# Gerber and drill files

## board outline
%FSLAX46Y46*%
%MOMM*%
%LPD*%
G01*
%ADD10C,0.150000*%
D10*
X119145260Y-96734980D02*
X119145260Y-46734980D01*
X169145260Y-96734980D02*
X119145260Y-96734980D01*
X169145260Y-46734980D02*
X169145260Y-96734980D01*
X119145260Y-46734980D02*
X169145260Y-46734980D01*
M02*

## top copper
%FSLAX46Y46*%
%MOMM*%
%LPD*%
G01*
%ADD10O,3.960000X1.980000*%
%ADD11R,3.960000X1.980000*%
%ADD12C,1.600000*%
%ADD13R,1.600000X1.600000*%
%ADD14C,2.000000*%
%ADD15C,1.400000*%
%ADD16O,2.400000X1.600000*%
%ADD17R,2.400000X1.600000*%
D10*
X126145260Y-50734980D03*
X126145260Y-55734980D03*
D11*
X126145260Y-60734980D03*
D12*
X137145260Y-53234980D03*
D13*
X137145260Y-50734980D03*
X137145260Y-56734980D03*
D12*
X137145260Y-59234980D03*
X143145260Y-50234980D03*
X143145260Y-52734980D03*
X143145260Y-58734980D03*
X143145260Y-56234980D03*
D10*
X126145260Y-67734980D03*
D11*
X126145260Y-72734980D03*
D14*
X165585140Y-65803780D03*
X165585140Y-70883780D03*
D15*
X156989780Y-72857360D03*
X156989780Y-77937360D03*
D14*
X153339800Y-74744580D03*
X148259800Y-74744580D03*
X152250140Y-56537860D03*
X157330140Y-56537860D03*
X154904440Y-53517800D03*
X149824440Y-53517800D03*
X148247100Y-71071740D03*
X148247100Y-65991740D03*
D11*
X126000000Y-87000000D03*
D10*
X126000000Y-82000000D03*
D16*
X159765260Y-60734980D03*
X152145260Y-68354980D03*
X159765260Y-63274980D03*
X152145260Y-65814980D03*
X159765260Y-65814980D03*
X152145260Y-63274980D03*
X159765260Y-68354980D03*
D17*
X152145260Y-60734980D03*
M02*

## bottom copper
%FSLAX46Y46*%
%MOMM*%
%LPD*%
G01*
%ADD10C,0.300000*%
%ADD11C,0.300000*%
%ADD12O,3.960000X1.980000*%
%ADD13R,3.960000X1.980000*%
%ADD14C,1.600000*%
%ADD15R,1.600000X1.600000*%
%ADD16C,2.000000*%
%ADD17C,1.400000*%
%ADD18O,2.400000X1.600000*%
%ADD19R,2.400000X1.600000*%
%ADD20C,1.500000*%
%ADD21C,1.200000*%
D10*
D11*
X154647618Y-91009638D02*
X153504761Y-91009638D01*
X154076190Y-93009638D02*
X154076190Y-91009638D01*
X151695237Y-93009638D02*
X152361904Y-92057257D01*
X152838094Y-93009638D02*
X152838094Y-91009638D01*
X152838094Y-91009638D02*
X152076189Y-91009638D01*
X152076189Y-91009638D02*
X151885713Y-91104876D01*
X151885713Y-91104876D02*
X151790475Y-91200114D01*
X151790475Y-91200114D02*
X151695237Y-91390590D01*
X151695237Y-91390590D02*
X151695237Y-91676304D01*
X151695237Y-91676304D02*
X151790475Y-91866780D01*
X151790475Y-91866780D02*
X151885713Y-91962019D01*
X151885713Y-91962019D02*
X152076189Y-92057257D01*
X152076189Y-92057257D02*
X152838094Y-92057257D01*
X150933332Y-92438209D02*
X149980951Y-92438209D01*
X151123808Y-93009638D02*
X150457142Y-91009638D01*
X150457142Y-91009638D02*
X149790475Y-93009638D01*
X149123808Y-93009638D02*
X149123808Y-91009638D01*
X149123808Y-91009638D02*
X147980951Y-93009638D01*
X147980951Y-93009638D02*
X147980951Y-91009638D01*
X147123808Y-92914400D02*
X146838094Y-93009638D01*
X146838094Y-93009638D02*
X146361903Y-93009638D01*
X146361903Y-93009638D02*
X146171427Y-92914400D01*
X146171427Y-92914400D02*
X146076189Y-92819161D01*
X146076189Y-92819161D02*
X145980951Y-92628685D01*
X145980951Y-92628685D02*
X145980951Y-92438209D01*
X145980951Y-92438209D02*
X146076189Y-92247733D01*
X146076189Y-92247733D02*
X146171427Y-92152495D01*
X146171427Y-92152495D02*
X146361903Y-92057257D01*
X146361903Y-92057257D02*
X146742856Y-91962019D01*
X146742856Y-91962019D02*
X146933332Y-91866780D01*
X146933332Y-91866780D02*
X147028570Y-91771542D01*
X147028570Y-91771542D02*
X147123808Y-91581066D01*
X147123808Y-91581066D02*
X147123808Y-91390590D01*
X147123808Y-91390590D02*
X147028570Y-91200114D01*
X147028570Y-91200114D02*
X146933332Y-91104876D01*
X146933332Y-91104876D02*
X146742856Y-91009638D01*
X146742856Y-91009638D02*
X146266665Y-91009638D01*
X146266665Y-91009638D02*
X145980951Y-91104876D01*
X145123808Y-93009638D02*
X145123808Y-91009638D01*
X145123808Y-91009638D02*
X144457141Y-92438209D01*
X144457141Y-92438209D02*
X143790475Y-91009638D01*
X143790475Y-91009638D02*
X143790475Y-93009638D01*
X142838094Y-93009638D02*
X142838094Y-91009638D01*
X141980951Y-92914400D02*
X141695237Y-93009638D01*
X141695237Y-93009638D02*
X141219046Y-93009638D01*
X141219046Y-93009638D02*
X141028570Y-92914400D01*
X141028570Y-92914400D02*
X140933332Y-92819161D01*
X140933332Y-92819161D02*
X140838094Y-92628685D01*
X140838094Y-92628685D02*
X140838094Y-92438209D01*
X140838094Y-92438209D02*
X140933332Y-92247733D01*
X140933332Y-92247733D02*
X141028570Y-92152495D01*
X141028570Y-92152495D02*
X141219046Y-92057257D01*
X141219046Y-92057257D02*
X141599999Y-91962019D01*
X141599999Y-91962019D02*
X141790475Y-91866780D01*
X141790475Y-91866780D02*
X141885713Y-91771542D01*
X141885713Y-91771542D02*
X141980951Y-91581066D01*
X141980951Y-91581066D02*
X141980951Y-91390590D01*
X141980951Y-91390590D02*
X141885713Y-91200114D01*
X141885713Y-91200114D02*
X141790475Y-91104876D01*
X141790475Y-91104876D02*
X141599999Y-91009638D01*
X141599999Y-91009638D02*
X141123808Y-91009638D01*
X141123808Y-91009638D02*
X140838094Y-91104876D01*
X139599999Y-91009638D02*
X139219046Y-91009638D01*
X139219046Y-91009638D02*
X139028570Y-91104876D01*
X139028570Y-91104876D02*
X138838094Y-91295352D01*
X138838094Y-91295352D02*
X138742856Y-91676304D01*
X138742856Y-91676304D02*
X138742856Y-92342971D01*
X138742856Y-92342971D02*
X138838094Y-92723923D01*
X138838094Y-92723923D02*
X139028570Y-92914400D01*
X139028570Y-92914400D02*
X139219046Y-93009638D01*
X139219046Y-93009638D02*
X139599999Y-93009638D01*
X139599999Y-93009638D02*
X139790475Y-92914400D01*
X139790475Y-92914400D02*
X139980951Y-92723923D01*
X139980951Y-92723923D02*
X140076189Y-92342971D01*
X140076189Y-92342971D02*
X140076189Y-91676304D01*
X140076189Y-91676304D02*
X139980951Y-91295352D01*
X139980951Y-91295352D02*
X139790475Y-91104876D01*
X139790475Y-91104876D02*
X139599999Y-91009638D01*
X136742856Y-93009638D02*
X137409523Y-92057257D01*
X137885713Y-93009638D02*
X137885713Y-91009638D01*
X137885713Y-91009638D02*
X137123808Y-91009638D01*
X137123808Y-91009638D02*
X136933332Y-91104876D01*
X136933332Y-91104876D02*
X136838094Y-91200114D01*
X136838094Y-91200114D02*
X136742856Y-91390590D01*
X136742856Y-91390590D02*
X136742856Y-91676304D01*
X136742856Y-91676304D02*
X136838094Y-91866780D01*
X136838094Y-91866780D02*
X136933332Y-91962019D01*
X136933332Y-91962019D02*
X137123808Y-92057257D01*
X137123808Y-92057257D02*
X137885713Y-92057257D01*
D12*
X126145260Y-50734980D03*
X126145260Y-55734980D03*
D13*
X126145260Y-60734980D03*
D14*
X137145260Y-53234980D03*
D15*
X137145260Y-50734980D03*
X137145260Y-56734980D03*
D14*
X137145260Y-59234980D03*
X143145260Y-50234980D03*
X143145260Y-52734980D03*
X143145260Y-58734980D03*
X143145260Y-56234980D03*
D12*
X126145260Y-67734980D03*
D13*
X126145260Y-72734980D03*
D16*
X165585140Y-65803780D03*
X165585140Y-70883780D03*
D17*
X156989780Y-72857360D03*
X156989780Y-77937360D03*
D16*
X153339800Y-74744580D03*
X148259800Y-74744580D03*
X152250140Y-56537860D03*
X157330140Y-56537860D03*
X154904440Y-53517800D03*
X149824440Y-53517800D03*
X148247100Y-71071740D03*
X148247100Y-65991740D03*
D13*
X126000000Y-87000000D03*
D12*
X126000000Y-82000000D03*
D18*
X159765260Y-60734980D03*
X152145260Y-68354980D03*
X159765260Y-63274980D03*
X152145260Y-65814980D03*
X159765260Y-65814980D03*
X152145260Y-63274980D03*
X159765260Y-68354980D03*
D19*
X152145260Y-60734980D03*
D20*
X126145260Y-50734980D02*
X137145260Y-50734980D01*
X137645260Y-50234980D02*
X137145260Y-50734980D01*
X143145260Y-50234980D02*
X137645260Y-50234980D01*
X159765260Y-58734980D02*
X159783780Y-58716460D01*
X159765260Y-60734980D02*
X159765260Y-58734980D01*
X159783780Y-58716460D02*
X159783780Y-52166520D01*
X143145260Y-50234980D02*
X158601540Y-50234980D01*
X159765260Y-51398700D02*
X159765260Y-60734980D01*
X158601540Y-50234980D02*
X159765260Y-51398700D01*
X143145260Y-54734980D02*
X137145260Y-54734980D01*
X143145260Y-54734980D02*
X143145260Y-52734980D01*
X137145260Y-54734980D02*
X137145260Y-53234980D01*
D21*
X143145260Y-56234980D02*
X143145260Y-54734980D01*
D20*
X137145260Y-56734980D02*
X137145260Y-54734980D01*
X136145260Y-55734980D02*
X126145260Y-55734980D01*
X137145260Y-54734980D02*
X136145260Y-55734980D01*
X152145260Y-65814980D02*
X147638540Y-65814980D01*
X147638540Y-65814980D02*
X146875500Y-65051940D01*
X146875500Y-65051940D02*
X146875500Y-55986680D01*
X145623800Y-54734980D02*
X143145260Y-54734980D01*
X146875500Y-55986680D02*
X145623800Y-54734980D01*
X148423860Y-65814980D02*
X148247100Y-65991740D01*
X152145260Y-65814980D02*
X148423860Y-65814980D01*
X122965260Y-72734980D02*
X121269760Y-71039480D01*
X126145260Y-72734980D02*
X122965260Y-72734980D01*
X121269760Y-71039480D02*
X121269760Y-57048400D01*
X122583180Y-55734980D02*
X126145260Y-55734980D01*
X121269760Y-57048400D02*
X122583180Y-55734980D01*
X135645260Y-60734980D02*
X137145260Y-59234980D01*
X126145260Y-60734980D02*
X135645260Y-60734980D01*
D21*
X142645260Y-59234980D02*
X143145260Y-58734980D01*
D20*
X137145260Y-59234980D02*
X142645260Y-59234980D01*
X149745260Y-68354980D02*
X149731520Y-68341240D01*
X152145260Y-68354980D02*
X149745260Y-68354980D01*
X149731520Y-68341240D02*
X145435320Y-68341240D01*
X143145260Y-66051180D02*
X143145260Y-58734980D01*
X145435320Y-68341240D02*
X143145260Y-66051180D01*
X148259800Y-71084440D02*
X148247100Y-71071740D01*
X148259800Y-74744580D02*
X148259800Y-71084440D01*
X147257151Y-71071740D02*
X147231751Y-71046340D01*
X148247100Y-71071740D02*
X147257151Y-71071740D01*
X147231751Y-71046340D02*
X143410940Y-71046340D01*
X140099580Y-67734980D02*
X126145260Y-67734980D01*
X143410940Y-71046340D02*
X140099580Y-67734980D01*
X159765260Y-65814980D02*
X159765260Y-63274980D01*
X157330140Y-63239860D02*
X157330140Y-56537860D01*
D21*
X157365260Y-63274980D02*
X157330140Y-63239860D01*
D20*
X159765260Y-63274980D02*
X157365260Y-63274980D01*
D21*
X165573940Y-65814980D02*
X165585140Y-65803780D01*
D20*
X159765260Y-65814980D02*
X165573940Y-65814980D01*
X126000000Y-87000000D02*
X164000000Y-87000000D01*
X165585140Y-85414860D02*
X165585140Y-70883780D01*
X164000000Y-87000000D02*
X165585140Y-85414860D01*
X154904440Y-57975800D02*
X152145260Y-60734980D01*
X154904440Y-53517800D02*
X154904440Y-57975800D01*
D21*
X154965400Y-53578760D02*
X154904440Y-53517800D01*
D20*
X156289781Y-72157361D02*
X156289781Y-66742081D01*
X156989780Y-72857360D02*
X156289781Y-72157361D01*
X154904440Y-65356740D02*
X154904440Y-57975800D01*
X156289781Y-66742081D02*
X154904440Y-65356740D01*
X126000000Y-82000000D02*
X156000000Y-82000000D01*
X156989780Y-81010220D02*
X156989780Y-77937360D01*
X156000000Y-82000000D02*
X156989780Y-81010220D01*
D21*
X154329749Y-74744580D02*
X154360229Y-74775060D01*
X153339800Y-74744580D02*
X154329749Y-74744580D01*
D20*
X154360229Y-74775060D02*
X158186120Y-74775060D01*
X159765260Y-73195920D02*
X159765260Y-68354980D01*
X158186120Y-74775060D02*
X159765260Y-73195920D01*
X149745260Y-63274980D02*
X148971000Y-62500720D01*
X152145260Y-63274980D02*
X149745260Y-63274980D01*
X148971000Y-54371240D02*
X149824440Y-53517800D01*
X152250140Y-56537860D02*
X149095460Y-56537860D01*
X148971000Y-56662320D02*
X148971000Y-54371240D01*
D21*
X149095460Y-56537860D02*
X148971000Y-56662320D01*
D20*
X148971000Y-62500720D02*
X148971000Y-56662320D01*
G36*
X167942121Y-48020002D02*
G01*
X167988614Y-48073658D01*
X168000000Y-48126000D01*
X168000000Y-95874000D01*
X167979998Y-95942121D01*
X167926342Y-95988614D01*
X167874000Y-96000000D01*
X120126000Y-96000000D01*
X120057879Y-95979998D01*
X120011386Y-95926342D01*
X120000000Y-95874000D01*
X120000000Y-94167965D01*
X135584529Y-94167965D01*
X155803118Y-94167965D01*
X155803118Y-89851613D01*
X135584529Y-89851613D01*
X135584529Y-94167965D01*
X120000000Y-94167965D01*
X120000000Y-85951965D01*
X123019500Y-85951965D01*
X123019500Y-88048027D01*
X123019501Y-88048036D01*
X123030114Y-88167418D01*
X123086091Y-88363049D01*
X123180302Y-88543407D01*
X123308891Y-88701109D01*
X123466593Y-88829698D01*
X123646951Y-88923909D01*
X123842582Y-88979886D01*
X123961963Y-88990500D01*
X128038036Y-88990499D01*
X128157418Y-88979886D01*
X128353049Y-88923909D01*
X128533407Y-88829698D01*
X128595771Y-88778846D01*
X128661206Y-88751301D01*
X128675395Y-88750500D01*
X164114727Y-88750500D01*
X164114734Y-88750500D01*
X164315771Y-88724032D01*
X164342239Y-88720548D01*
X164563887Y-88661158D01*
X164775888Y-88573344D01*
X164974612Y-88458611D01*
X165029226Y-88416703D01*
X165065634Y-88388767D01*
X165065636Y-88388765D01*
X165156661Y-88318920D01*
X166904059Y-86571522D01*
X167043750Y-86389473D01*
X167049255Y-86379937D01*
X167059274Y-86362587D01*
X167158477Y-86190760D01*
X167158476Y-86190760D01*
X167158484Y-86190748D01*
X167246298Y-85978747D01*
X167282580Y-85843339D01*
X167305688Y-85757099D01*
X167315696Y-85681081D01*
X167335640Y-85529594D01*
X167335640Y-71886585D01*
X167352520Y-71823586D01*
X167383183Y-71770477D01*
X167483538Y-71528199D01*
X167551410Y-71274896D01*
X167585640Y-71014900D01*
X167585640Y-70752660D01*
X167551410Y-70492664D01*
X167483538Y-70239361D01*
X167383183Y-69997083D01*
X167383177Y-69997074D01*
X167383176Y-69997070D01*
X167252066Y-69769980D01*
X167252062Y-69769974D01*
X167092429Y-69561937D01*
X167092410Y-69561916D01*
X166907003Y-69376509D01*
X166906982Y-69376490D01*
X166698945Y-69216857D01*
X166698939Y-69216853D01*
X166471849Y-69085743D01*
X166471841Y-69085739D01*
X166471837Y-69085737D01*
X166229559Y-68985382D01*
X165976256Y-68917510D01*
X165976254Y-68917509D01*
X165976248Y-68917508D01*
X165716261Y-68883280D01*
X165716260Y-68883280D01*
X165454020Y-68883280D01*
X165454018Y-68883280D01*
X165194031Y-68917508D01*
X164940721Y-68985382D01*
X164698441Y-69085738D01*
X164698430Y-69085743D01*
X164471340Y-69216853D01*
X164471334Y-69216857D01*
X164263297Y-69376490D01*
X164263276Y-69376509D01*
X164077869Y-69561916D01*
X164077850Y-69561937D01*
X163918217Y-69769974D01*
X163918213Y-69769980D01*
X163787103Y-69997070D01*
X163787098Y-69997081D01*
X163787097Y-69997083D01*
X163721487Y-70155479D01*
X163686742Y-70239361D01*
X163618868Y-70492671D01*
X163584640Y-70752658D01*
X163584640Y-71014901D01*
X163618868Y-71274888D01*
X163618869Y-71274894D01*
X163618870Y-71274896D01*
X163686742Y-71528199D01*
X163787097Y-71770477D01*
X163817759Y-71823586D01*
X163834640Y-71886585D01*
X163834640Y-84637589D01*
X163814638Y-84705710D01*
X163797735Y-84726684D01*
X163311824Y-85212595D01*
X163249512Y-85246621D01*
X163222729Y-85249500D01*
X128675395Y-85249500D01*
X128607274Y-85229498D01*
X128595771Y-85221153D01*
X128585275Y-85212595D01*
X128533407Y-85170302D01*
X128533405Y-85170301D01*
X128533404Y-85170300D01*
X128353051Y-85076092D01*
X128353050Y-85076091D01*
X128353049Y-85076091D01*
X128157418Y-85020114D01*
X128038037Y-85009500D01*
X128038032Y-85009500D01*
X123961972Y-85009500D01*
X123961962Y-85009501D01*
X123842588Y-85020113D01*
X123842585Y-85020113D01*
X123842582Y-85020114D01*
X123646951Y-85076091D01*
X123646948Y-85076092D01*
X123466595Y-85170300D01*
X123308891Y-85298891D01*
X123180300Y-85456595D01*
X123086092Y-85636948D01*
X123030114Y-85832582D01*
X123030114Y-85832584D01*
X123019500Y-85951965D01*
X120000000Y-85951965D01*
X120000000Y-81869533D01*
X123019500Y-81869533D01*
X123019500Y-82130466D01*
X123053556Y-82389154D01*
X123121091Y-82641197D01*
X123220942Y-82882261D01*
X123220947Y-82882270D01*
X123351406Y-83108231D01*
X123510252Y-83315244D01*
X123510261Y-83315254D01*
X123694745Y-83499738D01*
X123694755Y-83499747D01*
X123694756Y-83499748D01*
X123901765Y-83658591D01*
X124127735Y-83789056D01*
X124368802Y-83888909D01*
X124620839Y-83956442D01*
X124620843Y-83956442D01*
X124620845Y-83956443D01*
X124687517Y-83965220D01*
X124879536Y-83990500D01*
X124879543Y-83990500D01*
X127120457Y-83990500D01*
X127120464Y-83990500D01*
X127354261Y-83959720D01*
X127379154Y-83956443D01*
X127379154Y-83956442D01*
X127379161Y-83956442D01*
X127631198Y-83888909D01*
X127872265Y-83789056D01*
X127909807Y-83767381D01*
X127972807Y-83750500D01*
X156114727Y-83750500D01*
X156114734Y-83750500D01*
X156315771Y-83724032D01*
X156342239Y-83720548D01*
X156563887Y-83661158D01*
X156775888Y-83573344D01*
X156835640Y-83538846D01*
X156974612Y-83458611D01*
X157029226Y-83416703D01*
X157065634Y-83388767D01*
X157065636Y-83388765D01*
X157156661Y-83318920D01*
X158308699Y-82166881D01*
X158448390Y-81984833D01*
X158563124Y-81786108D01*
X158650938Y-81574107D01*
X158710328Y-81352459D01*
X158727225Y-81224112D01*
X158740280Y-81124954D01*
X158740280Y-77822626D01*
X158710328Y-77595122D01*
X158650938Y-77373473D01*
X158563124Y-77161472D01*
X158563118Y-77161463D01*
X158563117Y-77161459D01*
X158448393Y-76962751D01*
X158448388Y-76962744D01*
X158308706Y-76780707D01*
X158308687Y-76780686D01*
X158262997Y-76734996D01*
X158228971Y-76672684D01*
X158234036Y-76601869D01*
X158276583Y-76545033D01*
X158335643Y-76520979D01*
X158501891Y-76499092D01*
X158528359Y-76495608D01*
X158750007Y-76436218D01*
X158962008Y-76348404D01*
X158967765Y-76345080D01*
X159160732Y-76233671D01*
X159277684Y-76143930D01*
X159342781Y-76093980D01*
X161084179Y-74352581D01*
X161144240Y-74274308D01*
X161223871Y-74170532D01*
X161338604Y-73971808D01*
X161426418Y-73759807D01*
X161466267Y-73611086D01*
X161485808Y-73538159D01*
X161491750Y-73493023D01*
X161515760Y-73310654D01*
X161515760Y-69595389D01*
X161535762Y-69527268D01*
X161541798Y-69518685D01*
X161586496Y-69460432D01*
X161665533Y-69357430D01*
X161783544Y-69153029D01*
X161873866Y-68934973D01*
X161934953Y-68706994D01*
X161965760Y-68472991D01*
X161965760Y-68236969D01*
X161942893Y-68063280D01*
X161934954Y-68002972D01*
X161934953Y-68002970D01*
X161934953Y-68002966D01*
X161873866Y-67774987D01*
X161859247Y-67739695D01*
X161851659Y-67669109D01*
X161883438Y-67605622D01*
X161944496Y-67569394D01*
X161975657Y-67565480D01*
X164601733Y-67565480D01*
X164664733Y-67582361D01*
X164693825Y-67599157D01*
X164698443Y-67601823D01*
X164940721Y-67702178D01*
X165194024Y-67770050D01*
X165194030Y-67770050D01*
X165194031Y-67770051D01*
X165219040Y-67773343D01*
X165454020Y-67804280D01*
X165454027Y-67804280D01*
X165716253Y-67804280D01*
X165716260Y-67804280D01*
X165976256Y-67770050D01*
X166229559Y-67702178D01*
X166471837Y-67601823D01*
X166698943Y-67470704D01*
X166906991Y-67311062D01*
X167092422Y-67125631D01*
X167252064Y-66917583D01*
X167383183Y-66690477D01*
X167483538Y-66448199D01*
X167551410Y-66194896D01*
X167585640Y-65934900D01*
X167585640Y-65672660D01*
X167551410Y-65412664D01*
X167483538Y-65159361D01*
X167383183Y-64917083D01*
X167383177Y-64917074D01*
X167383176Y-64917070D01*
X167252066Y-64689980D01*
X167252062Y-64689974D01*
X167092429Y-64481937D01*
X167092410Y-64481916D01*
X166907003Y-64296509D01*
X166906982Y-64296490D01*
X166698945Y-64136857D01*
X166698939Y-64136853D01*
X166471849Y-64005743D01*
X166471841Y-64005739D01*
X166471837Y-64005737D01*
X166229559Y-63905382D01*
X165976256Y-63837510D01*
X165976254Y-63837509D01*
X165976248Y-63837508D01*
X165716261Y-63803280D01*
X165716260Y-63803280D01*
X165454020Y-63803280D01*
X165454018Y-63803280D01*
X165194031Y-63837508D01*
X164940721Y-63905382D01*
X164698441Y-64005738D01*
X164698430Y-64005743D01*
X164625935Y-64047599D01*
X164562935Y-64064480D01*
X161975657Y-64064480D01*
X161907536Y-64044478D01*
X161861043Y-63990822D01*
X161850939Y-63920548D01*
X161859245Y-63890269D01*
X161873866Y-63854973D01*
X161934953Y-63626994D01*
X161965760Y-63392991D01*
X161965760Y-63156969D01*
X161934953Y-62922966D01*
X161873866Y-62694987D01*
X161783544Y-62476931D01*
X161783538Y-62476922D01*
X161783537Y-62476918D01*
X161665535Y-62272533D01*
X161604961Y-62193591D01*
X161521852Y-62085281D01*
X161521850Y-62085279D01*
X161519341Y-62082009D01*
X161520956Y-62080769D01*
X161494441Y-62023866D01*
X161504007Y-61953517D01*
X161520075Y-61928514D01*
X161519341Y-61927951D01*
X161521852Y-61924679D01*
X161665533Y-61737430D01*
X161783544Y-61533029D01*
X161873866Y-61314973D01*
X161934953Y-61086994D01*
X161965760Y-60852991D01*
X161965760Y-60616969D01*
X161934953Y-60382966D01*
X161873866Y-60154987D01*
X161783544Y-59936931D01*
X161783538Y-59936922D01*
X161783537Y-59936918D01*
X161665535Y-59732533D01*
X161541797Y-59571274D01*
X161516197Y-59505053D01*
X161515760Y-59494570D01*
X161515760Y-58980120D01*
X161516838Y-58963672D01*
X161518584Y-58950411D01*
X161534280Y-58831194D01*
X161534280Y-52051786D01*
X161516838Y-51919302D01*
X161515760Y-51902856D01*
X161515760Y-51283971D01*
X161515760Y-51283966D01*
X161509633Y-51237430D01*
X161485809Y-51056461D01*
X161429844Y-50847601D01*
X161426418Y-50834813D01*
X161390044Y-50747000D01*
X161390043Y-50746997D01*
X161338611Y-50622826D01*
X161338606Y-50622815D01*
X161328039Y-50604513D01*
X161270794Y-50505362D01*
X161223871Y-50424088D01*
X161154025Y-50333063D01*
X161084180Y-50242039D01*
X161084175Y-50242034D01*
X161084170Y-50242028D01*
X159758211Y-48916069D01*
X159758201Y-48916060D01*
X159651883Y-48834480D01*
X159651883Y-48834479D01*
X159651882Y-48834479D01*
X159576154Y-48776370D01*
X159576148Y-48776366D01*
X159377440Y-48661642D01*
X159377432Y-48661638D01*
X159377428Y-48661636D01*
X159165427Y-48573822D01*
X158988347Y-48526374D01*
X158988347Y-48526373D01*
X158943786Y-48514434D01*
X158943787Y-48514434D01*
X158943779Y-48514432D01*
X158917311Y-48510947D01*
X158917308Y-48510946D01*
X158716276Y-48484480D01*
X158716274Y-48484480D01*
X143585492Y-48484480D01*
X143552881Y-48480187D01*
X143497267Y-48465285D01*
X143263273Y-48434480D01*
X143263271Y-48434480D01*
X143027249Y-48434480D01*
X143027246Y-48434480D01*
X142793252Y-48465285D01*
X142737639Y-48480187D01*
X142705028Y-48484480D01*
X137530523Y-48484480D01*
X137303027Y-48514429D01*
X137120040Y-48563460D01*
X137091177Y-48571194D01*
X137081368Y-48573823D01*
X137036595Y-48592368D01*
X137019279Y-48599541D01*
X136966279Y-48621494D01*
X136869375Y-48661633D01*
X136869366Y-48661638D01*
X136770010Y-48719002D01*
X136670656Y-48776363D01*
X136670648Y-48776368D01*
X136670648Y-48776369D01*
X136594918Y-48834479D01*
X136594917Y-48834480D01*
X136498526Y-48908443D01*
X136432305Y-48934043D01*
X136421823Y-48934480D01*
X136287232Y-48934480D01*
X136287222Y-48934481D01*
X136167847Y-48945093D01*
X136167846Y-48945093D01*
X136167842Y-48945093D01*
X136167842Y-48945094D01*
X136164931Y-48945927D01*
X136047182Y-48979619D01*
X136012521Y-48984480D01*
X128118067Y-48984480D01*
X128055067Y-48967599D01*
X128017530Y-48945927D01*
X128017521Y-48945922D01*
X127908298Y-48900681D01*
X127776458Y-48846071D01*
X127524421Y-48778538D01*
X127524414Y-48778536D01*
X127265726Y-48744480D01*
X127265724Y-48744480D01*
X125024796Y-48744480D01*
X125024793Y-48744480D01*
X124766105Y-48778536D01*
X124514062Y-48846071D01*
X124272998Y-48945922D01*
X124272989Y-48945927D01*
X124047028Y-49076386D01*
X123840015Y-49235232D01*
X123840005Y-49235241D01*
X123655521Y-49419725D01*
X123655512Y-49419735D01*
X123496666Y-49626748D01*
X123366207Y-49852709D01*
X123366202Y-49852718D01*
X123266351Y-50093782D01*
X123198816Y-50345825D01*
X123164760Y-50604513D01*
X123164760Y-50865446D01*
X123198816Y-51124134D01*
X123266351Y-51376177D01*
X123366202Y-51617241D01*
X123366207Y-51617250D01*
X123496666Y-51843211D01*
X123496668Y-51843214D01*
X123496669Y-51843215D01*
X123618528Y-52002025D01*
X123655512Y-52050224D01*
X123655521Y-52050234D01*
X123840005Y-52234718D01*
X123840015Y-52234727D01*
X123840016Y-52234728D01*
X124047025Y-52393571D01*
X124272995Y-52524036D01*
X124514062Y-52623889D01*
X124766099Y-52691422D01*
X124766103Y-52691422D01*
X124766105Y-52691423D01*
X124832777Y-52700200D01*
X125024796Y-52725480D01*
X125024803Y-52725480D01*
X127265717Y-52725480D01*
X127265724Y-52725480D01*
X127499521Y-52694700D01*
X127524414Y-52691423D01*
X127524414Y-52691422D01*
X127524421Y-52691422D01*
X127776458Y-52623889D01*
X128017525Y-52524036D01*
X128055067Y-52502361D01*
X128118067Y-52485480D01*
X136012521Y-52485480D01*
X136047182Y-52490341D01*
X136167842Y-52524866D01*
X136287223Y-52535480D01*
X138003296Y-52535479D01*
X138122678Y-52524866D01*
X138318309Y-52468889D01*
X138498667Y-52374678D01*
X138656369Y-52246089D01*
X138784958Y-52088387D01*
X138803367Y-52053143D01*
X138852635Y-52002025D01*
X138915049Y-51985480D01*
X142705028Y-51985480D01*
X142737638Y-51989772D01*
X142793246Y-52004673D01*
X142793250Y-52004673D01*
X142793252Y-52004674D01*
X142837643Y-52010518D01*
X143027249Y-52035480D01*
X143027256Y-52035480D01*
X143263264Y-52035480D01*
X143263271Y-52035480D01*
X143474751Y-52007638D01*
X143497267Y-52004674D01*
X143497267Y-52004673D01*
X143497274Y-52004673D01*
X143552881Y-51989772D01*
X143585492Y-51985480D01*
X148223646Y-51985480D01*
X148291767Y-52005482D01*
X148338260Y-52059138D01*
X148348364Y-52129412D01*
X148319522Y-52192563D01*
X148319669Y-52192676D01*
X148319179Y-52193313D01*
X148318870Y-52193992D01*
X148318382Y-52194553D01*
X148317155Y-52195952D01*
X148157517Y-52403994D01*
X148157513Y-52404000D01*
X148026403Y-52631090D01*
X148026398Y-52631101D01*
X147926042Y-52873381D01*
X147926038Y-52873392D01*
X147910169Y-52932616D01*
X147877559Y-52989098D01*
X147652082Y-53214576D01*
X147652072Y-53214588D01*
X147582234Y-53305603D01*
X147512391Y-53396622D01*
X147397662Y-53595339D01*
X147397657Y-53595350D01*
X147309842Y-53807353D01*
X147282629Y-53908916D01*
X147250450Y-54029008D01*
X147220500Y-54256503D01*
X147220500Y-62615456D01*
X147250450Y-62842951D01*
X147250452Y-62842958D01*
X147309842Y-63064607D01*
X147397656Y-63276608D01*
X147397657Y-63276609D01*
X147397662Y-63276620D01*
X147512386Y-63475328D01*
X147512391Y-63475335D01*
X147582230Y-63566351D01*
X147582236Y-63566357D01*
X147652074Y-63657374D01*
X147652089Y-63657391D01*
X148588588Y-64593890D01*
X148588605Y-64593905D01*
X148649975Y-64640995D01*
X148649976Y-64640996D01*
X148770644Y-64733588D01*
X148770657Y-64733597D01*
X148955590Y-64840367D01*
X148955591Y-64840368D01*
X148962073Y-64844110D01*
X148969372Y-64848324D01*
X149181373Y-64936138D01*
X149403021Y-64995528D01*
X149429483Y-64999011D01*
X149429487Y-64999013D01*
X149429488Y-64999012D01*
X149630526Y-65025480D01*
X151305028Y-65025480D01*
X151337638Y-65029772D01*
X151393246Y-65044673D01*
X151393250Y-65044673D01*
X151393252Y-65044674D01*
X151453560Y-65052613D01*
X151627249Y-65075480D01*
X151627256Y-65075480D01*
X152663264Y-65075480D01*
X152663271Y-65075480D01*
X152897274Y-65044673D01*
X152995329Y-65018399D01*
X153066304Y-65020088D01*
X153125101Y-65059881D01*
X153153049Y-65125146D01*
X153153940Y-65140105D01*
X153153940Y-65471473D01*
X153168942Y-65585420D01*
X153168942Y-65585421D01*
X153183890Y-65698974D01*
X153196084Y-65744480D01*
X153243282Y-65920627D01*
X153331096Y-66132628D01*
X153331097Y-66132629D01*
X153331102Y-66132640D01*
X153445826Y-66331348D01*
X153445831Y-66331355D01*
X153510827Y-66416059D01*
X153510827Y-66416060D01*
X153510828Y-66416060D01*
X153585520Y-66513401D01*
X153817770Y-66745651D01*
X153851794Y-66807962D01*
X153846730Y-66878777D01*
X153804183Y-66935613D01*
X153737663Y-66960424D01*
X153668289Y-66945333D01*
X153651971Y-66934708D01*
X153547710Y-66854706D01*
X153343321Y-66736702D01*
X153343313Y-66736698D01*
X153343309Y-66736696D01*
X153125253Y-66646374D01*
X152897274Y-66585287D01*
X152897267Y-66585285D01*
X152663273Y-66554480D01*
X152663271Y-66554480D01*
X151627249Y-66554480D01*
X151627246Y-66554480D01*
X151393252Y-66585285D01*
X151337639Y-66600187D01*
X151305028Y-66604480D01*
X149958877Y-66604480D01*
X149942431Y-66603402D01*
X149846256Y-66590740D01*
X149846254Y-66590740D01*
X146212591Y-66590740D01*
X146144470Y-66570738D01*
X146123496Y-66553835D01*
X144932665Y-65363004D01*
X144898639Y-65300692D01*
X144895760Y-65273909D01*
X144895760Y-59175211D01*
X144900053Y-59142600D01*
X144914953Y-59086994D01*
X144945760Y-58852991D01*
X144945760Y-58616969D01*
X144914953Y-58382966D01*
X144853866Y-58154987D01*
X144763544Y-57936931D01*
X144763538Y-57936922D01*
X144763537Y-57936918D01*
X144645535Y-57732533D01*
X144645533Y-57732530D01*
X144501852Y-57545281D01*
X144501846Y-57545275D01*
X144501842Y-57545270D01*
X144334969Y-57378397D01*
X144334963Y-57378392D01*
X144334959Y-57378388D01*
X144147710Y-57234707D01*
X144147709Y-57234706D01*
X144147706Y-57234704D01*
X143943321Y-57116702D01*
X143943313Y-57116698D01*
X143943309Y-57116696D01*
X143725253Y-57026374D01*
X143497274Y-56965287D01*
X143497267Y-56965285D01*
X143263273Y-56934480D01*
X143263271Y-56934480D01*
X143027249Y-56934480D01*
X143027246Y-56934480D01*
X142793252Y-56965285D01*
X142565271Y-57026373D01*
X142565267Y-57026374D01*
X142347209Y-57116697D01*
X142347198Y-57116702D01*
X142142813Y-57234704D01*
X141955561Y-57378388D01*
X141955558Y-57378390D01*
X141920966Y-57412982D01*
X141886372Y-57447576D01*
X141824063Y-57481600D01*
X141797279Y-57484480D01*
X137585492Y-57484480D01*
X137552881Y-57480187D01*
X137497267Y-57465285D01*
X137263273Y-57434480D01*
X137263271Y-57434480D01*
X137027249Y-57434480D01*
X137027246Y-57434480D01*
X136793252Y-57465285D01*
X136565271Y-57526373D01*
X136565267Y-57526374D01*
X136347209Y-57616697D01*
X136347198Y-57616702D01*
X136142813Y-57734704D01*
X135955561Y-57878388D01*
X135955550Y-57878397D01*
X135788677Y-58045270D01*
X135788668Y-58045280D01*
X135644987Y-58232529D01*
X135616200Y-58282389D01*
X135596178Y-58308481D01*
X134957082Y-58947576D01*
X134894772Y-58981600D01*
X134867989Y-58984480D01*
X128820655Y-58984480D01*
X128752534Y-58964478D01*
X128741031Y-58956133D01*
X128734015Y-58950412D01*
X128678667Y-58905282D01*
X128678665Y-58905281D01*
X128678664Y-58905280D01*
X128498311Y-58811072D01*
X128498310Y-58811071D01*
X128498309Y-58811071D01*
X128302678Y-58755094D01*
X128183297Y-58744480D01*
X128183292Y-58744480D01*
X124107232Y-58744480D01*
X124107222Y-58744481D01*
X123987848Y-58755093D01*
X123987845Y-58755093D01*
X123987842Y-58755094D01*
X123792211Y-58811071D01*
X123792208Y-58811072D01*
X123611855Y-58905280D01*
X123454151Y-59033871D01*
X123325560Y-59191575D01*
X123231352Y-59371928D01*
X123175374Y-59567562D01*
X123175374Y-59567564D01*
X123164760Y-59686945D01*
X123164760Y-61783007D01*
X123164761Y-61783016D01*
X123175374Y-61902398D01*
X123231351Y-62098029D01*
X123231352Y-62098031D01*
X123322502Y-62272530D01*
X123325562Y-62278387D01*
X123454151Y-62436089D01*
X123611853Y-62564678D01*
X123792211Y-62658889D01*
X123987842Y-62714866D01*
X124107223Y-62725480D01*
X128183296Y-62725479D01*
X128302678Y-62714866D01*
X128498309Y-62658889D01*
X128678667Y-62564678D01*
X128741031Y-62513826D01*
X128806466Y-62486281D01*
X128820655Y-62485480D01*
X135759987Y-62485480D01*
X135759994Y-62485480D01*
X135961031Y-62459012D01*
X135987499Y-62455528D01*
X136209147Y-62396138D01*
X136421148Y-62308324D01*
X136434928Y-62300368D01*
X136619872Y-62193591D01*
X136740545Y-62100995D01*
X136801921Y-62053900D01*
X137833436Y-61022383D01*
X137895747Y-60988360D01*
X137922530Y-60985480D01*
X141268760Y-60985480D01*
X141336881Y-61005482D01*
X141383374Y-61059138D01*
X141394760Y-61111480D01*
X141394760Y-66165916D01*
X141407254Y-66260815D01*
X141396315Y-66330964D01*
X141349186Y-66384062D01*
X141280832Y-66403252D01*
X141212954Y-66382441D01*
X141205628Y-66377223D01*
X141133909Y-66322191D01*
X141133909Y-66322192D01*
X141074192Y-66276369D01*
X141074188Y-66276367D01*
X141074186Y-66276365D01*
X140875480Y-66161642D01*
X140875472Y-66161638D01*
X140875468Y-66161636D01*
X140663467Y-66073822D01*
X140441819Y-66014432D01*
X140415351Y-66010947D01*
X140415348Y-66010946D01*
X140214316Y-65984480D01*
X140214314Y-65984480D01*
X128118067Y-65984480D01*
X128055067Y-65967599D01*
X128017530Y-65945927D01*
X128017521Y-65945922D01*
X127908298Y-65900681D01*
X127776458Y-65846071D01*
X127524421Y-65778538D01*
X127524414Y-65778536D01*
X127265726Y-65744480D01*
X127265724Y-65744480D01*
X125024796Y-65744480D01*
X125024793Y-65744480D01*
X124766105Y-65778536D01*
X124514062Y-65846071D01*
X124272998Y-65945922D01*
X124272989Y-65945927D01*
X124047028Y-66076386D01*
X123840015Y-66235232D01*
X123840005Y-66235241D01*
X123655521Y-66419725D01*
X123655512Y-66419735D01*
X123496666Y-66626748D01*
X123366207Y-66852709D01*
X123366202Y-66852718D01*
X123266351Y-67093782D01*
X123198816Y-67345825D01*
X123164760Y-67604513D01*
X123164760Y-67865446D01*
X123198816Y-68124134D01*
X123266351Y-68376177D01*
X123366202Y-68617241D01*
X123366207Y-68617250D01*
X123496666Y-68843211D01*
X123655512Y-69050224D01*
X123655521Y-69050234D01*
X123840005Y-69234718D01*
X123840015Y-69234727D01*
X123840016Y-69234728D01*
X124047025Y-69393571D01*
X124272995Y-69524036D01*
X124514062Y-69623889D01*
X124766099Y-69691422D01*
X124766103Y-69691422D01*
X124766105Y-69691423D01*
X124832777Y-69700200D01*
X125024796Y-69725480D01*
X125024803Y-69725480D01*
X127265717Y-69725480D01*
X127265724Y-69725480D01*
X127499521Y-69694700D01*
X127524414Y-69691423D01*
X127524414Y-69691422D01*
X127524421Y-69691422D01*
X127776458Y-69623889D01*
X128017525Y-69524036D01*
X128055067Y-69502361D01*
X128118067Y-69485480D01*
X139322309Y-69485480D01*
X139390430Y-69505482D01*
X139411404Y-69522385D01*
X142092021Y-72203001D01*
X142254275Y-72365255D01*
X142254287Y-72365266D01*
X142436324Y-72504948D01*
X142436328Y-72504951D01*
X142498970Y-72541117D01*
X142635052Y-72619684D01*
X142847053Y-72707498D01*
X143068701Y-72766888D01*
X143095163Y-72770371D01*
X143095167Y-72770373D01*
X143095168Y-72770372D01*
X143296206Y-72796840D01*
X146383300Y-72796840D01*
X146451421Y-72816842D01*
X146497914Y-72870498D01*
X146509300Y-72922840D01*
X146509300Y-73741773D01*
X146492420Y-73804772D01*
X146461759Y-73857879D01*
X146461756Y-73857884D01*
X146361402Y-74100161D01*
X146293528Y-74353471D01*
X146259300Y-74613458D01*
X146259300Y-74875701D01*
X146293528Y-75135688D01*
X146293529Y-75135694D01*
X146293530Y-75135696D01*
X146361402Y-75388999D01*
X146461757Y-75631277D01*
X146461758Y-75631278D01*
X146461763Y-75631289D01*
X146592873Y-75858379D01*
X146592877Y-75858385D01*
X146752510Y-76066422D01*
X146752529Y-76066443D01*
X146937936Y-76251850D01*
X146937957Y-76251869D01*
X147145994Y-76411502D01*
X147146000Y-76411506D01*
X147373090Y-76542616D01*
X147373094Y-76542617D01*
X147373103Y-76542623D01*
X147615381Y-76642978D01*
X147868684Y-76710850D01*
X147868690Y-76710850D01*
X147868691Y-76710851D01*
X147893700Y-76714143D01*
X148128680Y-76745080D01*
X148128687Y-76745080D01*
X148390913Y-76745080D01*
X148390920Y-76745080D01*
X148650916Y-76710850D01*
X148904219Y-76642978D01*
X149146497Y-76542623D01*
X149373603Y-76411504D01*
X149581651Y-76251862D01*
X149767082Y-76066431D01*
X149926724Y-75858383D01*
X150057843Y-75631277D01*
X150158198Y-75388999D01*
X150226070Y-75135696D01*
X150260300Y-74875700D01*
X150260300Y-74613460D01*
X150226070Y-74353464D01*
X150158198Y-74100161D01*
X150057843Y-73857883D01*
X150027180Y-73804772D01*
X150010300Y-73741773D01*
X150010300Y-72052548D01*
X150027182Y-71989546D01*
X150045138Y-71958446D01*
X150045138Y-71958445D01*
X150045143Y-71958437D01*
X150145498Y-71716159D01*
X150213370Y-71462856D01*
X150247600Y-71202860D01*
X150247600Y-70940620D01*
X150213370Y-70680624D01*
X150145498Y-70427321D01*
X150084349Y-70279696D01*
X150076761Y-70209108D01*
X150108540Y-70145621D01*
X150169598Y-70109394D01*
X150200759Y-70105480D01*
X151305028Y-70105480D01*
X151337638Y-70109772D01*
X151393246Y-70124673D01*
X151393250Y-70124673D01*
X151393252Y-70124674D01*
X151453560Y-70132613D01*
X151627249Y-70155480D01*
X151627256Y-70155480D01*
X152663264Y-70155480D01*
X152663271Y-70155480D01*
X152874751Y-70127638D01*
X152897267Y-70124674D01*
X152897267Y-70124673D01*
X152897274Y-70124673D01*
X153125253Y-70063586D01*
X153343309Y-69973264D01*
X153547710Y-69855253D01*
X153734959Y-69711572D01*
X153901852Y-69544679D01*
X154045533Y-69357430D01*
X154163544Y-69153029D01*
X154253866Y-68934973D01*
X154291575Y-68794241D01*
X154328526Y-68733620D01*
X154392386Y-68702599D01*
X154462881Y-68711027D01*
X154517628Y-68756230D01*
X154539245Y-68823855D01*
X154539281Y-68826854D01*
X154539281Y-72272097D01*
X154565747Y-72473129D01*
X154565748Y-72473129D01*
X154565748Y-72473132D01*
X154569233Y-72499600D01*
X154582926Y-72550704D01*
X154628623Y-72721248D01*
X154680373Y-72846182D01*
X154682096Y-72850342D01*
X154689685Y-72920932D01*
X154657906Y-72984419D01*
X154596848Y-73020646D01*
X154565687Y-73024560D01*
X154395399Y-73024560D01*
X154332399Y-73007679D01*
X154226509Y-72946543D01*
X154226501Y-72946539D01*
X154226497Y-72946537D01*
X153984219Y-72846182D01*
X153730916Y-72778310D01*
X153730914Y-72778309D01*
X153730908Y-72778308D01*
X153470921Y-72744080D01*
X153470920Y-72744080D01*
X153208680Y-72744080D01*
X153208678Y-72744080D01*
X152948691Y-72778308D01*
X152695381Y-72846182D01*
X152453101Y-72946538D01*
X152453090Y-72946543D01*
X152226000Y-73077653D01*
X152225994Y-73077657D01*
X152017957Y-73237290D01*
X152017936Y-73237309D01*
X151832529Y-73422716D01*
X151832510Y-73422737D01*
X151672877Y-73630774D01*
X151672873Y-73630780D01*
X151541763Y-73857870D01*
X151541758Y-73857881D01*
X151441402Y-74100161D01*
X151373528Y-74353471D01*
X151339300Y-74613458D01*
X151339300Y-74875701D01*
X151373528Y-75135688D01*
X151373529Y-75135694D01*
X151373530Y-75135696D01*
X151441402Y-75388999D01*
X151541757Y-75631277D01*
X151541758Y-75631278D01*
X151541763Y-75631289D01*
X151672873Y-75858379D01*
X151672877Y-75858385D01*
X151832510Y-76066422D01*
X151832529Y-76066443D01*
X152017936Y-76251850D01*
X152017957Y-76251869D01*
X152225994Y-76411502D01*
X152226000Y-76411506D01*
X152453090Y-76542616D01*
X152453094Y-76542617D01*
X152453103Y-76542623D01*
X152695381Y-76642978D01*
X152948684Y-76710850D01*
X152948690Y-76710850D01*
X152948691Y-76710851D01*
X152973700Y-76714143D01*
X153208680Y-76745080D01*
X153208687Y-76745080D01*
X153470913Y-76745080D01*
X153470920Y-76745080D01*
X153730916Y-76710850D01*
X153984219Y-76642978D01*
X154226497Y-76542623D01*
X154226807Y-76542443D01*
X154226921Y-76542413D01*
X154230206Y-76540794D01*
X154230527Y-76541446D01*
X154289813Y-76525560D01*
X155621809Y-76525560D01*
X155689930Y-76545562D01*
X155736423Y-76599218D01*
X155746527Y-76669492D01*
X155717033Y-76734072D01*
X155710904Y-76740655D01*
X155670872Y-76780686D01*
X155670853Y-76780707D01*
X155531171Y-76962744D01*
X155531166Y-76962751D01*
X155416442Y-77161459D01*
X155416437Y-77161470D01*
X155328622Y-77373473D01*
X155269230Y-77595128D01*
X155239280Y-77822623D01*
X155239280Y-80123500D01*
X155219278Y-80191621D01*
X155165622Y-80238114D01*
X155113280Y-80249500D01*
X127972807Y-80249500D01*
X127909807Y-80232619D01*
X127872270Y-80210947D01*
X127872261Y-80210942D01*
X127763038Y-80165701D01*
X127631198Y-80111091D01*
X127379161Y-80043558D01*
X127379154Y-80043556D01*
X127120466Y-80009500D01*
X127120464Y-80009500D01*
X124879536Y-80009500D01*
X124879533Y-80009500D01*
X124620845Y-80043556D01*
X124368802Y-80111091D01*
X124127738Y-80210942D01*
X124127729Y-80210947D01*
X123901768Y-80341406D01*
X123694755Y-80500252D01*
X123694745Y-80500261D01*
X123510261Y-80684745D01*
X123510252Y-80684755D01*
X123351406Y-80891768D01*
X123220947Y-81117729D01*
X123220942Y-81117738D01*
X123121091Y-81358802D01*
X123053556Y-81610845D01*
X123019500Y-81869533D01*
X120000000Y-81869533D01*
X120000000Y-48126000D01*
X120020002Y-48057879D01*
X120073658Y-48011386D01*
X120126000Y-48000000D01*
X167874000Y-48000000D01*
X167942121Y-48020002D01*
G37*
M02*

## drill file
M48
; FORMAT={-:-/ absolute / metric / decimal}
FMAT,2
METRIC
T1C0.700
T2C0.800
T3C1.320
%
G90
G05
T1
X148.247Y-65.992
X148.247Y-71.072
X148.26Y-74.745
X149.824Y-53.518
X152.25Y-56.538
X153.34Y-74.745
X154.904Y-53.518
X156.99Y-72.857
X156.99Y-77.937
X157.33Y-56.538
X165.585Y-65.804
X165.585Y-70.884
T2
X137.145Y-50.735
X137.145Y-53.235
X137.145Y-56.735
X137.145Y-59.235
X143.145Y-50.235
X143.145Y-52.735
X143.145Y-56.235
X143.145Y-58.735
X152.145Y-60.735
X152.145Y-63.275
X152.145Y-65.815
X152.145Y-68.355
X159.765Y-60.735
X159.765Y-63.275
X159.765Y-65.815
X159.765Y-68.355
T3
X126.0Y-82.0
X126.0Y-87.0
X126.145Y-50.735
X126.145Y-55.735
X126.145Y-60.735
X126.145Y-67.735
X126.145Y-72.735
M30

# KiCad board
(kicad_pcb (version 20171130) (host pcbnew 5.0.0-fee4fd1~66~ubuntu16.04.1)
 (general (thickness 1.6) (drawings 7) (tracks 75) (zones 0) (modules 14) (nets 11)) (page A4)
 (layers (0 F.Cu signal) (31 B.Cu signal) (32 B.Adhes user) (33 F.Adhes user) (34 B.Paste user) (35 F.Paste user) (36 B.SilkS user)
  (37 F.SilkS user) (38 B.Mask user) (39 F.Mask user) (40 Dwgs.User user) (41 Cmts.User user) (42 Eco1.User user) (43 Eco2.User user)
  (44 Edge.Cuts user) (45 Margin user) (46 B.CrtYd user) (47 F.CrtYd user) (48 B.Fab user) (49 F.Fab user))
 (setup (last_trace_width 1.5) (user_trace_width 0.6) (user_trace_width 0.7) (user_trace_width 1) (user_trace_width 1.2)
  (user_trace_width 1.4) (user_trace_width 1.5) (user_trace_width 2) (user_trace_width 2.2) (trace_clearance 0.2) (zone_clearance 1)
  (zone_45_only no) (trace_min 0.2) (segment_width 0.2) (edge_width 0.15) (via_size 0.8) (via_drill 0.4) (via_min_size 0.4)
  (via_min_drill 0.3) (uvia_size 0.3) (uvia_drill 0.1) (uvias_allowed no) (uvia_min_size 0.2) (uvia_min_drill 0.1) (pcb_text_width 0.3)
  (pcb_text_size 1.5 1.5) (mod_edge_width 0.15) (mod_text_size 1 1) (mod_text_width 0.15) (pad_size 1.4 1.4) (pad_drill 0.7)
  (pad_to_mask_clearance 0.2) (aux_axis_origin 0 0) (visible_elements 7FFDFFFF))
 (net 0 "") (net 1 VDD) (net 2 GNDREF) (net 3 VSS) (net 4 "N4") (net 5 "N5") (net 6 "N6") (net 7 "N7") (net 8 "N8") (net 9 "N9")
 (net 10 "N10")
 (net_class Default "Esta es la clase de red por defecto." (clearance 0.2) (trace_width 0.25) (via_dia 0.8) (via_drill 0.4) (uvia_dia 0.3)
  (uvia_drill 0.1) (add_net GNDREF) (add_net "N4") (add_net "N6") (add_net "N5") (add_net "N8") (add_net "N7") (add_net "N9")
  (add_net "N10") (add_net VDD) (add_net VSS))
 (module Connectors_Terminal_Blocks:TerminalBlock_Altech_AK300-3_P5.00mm (layer F.Cu) (at 126.14526 60.73498 90)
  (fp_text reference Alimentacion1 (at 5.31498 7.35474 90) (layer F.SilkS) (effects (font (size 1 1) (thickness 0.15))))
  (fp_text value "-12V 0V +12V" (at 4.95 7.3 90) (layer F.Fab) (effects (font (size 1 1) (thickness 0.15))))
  (pad 3 thru_hole oval (at 10 0 90) (size 1.98 3.96) (drill 1.32) (layers *.Cu *.Mask) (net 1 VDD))
  (pad 2 thru_hole oval (at 5 0 90) (size 1.98 3.96) (drill 1.32) (layers *.Cu *.Mask) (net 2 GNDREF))
  (pad 1 thru_hole rect (at 0 0 90) (size 1.98 3.96) (drill 1.32) (layers *.Cu *.Mask) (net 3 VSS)))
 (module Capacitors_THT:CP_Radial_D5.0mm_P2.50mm (layer F.Cu) (at 137.14526 50.73498 270)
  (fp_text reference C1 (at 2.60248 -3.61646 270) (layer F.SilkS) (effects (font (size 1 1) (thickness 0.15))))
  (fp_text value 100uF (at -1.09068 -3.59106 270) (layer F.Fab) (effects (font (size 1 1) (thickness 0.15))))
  (pad 2 thru_hole circle (at 2.5 0 270) (size 1.6 1.6) (drill 0.8) (layers *.Cu *.Mask) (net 2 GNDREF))
  (pad 1 thru_hole rect (at 0 0 270) (size 1.6 1.6) (drill 0.8) (layers *.Cu *.Mask) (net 1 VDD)))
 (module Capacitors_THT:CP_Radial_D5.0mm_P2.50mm (layer F.Cu) (at 137.14526 56.73498 270)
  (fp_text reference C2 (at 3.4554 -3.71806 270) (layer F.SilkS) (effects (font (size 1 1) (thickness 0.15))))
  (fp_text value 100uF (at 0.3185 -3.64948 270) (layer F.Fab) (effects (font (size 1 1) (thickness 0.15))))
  (pad 1 thru_hole rect (at 0 0 270) (size 1.6 1.6) (drill 0.8) (layers *.Cu *.Mask) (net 2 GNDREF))
  (pad 2 thru_hole circle (at 2.5 0 270) (size 1.6 1.6) (drill 0.8) (layers *.Cu *.Mask) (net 3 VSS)))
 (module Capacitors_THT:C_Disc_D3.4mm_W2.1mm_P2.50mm (layer F.Cu) (at 143.14526 52.73498 90)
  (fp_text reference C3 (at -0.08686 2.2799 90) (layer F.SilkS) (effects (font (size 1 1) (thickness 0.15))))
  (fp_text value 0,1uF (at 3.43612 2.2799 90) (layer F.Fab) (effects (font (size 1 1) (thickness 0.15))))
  (pad 2 thru_hole circle (at 2.5 0 90) (size 1.6 1.6) (drill 0.8) (layers *.Cu *.Mask) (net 1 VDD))
  (pad 1 thru_hole circle (at 0 0 90) (size 1.6 1.6) (drill 0.8) (layers *.Cu *.Mask) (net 2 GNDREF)))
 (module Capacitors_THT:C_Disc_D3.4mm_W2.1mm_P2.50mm (layer F.Cu) (at 143.14526 58.73498 90)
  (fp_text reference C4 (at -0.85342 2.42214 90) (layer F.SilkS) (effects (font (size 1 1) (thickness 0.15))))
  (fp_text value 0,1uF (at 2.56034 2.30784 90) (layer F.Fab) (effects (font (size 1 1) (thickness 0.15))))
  (pad 1 thru_hole circle (at 0 0 90) (size 1.6 1.6) (drill 0.8) (layers *.Cu *.Mask) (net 3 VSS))
  (pad 2 thru_hole circle (at 2.5 0 90) (size 1.6 1.6) (drill 0.8) (layers *.Cu *.Mask) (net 2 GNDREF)))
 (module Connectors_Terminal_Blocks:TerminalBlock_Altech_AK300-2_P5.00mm (layer F.Cu) (at 126.14526 72.73498 90)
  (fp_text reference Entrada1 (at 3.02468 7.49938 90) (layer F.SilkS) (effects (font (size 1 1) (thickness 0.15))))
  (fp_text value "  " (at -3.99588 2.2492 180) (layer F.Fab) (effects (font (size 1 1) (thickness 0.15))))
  (pad 2 thru_hole oval (at 5 0 90) (size 1.98 3.96) (drill 1.32) (layers *.Cu *.Mask) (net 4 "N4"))
  (pad 1 thru_hole rect (at 0 0 90) (size 1.98 3.96) (drill 1.32) (layers *.Cu *.Mask) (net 2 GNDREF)))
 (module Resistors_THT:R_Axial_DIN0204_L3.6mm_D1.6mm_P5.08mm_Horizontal (layer F.Cu) (at 165.58514 70.88378 90)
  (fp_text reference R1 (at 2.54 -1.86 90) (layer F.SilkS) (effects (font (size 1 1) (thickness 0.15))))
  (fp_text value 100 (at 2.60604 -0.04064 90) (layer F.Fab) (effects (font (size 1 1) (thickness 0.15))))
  (pad 2 thru_hole circle (at 5.08 0 90) (size 2 2) (drill 0.7) (layers *.Cu *.Mask) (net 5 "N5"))
  (pad 1 thru_hole circle (at 0 0 90) (size 2 2) (drill 0.7) (layers *.Cu *.Mask) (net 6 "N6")))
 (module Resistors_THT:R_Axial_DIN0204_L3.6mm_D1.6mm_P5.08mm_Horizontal (layer F.Cu) (at 156.98978 77.93736 90)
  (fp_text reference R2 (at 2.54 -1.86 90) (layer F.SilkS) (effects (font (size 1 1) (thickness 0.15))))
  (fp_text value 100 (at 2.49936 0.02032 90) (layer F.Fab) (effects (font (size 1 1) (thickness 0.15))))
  (pad 2 thru_hole circle (at 5.08 0 90) (size 1.4 1.4) (drill 0.7) (layers *.Cu *.Mask) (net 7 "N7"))
  (pad 1 thru_hole circle (at 0 0 90) (size 1.4 1.4) (drill 0.7) (layers *.Cu *.Mask) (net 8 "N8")))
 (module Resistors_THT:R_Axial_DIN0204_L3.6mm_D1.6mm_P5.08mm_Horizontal (layer F.Cu) (at 153.3398 74.74458 180)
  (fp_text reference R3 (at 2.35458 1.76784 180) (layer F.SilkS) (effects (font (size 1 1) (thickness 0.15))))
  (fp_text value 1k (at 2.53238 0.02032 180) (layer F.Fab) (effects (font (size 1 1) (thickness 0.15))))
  (pad 1 thru_hole circle (at 0 0 180) (size 2 2) (drill 0.7) (layers *.Cu *.Mask) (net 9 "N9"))
  (pad 2 thru_hole circle (at 5.08 0 180) (size 2 2) (drill 0.7) (layers *.Cu *.Mask) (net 4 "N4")))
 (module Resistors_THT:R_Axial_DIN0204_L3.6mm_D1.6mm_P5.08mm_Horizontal (layer F.Cu) (at 152.25014 56.53786)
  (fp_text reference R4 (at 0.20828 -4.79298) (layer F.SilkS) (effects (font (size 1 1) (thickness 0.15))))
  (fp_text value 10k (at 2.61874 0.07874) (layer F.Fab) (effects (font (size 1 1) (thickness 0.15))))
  (pad 1 thru_hole circle (at 0 0) (size 2 2) (drill 0.7) (layers *.Cu *.Mask) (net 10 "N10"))
  (pad 2 thru_hole circle (at 5.08 0) (size 2 2) (drill 0.7) (layers *.Cu *.Mask) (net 5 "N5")))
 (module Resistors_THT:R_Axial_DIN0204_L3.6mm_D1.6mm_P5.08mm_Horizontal (layer F.Cu) (at 154.90444 53.5178 180)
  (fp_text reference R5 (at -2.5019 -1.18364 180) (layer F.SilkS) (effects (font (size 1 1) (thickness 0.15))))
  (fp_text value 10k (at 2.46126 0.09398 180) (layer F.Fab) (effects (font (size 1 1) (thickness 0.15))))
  (pad 1 thru_hole circle (at 0 0 180) (size 2 2) (drill 0.7) (layers *.Cu *.Mask) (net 7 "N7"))
  (pad 2 thru_hole circle (at 5.08 0 180) (size 2 2) (drill 0.7) (layers *.Cu *.Mask) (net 10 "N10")))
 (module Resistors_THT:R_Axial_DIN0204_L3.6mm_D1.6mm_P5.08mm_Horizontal (layer F.Cu) (at 148.2471 65.99174 270)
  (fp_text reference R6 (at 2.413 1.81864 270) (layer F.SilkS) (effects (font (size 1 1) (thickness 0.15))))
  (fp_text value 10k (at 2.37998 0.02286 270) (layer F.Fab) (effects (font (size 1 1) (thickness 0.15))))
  (pad 2 thru_hole circle (at 5.08 0 270) (size 2 2) (drill 0.7) (layers *.Cu *.Mask) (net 4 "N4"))
  (pad 1 thru_hole circle (at 0 0 270) (size 2 2) (drill 0.7) (layers *.Cu *.Mask) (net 2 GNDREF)))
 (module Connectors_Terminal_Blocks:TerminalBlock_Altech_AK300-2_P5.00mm (layer F.Cu) (at 126 87 90)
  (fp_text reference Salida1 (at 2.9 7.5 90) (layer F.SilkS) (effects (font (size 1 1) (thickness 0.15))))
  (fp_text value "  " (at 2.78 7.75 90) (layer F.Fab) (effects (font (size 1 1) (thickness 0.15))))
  (pad 1 thru_hole rect (at 0 0 90) (size 1.98 3.96) (drill 1.32) (layers *.Cu *.Mask) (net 6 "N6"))
  (pad 2 thru_hole oval (at 5 0 90) (size 1.98 3.96) (drill 1.32) (layers *.Cu *.Mask) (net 8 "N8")))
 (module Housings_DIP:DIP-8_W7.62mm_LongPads (layer F.Cu) (at 152.14526 60.73498)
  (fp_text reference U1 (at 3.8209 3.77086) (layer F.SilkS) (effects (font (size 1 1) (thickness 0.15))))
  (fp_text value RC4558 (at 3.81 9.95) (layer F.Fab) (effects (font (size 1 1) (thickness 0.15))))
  (pad 8 thru_hole oval (at 7.62 0) (size 2.4 1.6) (drill 0.8) (layers *.Cu *.Mask) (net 1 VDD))
  (pad 4 thru_hole oval (at 0 7.62) (size 2.4 1.6) (drill 0.8) (layers *.Cu *.Mask) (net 3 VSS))
  (pad 7 thru_hole oval (at 7.62 2.54) (size 2.4 1.6) (drill 0.8) (layers *.Cu *.Mask) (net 5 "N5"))
  (pad 3 thru_hole oval (at 0 5.08) (size 2.4 1.6) (drill 0.8) (layers *.Cu *.Mask) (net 2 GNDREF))
  (pad 6 thru_hole oval (at 7.62 5.08) (size 2.4 1.6) (drill 0.8) (layers *.Cu *.Mask) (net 5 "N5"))
  (pad 2 thru_hole oval (at 0 2.54) (size 2.4 1.6) (drill 0.8) (layers *.Cu *.Mask) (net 10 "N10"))
  (pad 5 thru_hole oval (at 7.62 7.62) (size 2.4 1.6) (drill 0.8) (layers *.Cu *.Mask) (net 9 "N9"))
  (pad 1 thru_hole rect (at 0 0) (size 2.4 1.6) (drill 0.8) (layers *.Cu *.Mask) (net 7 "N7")))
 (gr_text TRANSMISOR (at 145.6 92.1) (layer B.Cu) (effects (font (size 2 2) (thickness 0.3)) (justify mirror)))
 (gr_line (start 119.14526 96.73498) (end 119.14526 46.73498) (layer Edge.Cuts) (width 0.15))
 (gr_line (start 169.14526 96.73498) (end 119.14526 96.73498) (layer Edge.Cuts) (width 0.15))
 (gr_line (start 169.14526 46.73498) (end 169.14526 96.73498) (layer Edge.Cuts) (width 0.15))
 (gr_line (start 119.14526 46.73498) (end 169.14526 46.73498) (layer Edge.Cuts) (width 0.15))
 (segment (start 126.14526 50.73498) (end 137.14526 50.73498) (width 1.5) (layer B.Cu) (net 1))
 (segment (start 137.64526 50.23498) (end 137.14526 50.73498) (width 1.5) (layer B.Cu) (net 1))
 (segment (start 143.14526 50.23498) (end 137.64526 50.23498) (width 1.5) (layer B.Cu) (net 1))
 (segment (start 159.76526 58.73498) (end 159.78378 58.71646) (width 1.5) (layer B.Cu) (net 1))
 (segment (start 159.76526 60.73498) (end 159.76526 58.73498) (width 1.5) (layer B.Cu) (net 1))
 (segment (start 159.78378 58.71646) (end 159.78378 52.16652) (width 1.5) (layer B.Cu) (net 1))
 (segment (start 143.14526 50.23498) (end 158.60154 50.23498) (width 1.5) (layer B.Cu) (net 1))
 (segment (start 159.76526 51.3987) (end 159.76526 60.73498) (width 1.5) (layer B.Cu) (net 1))
 (segment (start 158.60154 50.23498) (end 159.76526 51.3987) (width 1.5) (layer B.Cu) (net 1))
 (segment (start 143.14526 54.73498) (end 137.14526 54.73498) (width 1.5) (layer B.Cu) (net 2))
 (segment (start 143.14526 54.73498) (end 143.14526 52.73498) (width 1.5) (layer B.Cu) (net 2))
 (segment (start 137.14526 54.73498) (end 137.14526 53.23498) (width 1.5) (layer B.Cu) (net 2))
 (segment (start 143.14526 56.23498) (end 143.14526 54.73498) (width 1.2) (layer B.Cu) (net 2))
 (segment (start 137.14526 56.73498) (end 137.14526 54.73498) (width 1.5) (layer B.Cu) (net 2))
 (segment (start 136.14526 55.73498) (end 126.14526 55.73498) (width 1.5) (layer B.Cu) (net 2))
 (segment (start 137.14526 54.73498) (end 136.14526 55.73498) (width 1.5) (layer B.Cu) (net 2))
 (segment (start 152.14526 65.81498) (end 147.63854 65.81498) (width 1.5) (layer B.Cu) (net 2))
 (segment (start 147.63854 65.81498) (end 146.8755 65.05194) (width 1.5) (layer B.Cu) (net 2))
 (segment (start 146.8755 65.05194) (end 146.8755 55.98668) (width 1.5) (layer B.Cu) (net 2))
 (segment (start 145.6238 54.73498) (end 143.14526 54.73498) (width 1.5) (layer B.Cu) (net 2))
 (segment (start 146.8755 55.98668) (end 145.6238 54.73498) (width 1.5) (layer B.Cu) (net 2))
 (segment (start 148.42386 65.81498) (end 148.2471 65.99174) (width 1.5) (layer B.Cu) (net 2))
 (segment (start 152.14526 65.81498) (end 148.42386 65.81498) (width 1.5) (layer B.Cu) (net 2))
 (segment (start 122.96526 72.73498) (end 121.26976 71.03948) (width 1.5) (layer B.Cu) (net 2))
 (segment (start 126.14526 72.73498) (end 122.96526 72.73498) (width 1.5) (layer B.Cu) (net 2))
 (segment (start 121.26976 71.03948) (end 121.26976 57.0484) (width 1.5) (layer B.Cu) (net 2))
 (segment (start 122.58318 55.73498) (end 126.14526 55.73498) (width 1.5) (layer B.Cu) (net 2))
 (segment (start 121.26976 57.0484) (end 122.58318 55.73498) (width 1.5) (layer B.Cu) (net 2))
 (segment (start 135.64526 60.73498) (end 137.14526 59.23498) (width 1.5) (layer B.Cu) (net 3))
 (segment (start 126.14526 60.73498) (end 135.64526 60.73498) (width 1.5) (layer B.Cu) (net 3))
 (segment (start 142.64526 59.23498) (end 143.14526 58.73498) (width 1.2) (layer B.Cu) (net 3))
 (segment (start 137.14526 59.23498) (end 142.64526 59.23498) (width 1.5) (layer B.Cu) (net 3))
 (segment (start 149.74526 68.35498) (end 149.73152 68.34124) (width 1.5) (layer B.Cu) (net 3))
 (segment (start 152.14526 68.35498) (end 149.74526 68.35498) (width 1.5) (layer B.Cu) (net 3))
 (segment (start 149.73152 68.34124) (end 145.43532 68.34124) (width 1.5) (layer B.Cu) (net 3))
 (segment (start 143.14526 66.05118) (end 143.14526 58.73498) (width 1.5) (layer B.Cu) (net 3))
 (segment (start 145.43532 68.34124) (end 143.14526 66.05118) (width 1.5) (layer B.Cu) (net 3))
 (segment (start 148.2598 71.08444) (end 148.2471 71.07174) (width 1.5) (layer B.Cu) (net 4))
 (segment (start 148.2598 74.74458) (end 148.2598 71.08444) (width 1.5) (layer B.Cu) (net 4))
 (segment (start 147.257151 71.07174) (end 147.231751 71.04634) (width 1.5) (layer B.Cu) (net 4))
 (segment (start 148.2471 71.07174) (end 147.257151 71.07174) (width 1.5) (layer B.Cu) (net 4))
 (segment (start 147.231751 71.04634) (end 143.41094 71.04634) (width 1.5) (layer B.Cu) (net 4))
 (segment (start 140.09958 67.73498) (end 126.14526 67.73498) (width 1.5) (layer B.Cu) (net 4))
 (segment (start 143.41094 71.04634) (end 140.09958 67.73498) (width 1.5) (layer B.Cu) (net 4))
 (segment (start 159.76526 65.81498) (end 159.76526 63.27498) (width 1.5) (layer B.Cu) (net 5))
 (segment (start 157.33014 63.23986) (end 157.33014 56.53786) (width 1.5) (layer B.Cu) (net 5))
 (segment (start 157.36526 63.27498) (end 157.33014 63.23986) (width 1.2) (layer B.Cu) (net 5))
 (segment (start 159.76526 63.27498) (end 157.36526 63.27498) (width 1.5) (layer B.Cu) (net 5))
 (segment (start 165.57394 65.81498) (end 165.58514 65.80378) (width 1.2) (layer B.Cu) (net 5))
 (segment (start 159.76526 65.81498) (end 165.57394 65.81498) (width 1.5) (layer B.Cu) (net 5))
 (segment (start 126 87) (end 164 87) (width 1.5) (layer B.Cu) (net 6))
 (segment (start 165.58514 85.41486) (end 165.58514 70.88378) (width 1.5) (layer B.Cu) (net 6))
 (segment (start 164 87) (end 165.58514 85.41486) (width 1.5) (layer B.Cu) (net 6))
 (segment (start 154.90444 57.9758) (end 152.14526 60.73498) (width 1.5) (layer B.Cu) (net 7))
 (segment (start 154.90444 53.5178) (end 154.90444 57.9758) (width 1.5) (layer B.Cu) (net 7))
 (segment (start 154.9654 53.57876) (end 154.90444 53.5178) (width 1.2) (layer B.Cu) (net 7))
 (segment (start 156.289781 72.157361) (end 156.289781 66.742081) (width 1.5) (layer B.Cu) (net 7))
 (segment (start 156.98978 72.85736) (end 156.289781 72.157361) (width 1.5) (layer B.Cu) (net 7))
 (segment (start 154.90444 65.35674) (end 154.90444 57.9758) (width 1.5) (layer B.Cu) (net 7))
 (segment (start 156.289781 66.742081) (end 154.90444 65.35674) (width 1.5) (layer B.Cu) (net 7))
 (segment (start 126 82) (end 156 82) (width 1.5) (layer B.Cu) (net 8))
 (segment (start 156.98978 81.01022) (end 156.98978 77.93736) (width 1.5) (layer B.Cu) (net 8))
 (segment (start 156 82) (end 156.98978 81.01022) (width 1.5) (layer B.Cu) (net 8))
 (segment (start 154.329749 74.74458) (end 154.360229 74.77506) (width 1.2) (layer B.Cu) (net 9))
 (segment (start 153.3398 74.74458) (end 154.329749 74.74458) (width 1.2) (layer B.Cu) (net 9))
 (segment (start 154.360229 74.77506) (end 158.18612 74.77506) (width 1.5) (layer B.Cu) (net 9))
 (segment (start 159.76526 73.19592) (end 159.76526 68.35498) (width 1.5) (layer B.Cu) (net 9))
 (segment (start 158.18612 74.77506) (end 159.76526 73.19592) (width 1.5) (layer B.Cu) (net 9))
 (segment (start 149.74526 63.27498) (end 148.971 62.50072) (width 1.5) (layer B.Cu) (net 10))
 (segment (start 152.14526 63.27498) (end 149.74526 63.27498) (width 1.5) (layer B.Cu) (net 10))
 (segment (start 148.971 54.37124) (end 149.82444 53.5178) (width 1.5) (layer B.Cu) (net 10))
 (segment (start 152.25014 56.53786) (end 149.09546 56.53786) (width 1.5) (layer B.Cu) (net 10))
 (segment (start 148.971 56.66232) (end 148.971 54.37124) (width 1.5) (layer B.Cu) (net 10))
 (segment (start 149.09546 56.53786) (end 148.971 56.66232) (width 1.2) (layer B.Cu) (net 10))
 (segment (start 148.971 62.50072) (end 148.971 56.66232) (width 1.5) (layer B.Cu) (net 10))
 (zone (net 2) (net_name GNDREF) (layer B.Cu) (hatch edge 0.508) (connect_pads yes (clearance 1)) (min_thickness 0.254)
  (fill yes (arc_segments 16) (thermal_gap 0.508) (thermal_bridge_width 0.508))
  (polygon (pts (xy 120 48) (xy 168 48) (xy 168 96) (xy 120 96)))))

